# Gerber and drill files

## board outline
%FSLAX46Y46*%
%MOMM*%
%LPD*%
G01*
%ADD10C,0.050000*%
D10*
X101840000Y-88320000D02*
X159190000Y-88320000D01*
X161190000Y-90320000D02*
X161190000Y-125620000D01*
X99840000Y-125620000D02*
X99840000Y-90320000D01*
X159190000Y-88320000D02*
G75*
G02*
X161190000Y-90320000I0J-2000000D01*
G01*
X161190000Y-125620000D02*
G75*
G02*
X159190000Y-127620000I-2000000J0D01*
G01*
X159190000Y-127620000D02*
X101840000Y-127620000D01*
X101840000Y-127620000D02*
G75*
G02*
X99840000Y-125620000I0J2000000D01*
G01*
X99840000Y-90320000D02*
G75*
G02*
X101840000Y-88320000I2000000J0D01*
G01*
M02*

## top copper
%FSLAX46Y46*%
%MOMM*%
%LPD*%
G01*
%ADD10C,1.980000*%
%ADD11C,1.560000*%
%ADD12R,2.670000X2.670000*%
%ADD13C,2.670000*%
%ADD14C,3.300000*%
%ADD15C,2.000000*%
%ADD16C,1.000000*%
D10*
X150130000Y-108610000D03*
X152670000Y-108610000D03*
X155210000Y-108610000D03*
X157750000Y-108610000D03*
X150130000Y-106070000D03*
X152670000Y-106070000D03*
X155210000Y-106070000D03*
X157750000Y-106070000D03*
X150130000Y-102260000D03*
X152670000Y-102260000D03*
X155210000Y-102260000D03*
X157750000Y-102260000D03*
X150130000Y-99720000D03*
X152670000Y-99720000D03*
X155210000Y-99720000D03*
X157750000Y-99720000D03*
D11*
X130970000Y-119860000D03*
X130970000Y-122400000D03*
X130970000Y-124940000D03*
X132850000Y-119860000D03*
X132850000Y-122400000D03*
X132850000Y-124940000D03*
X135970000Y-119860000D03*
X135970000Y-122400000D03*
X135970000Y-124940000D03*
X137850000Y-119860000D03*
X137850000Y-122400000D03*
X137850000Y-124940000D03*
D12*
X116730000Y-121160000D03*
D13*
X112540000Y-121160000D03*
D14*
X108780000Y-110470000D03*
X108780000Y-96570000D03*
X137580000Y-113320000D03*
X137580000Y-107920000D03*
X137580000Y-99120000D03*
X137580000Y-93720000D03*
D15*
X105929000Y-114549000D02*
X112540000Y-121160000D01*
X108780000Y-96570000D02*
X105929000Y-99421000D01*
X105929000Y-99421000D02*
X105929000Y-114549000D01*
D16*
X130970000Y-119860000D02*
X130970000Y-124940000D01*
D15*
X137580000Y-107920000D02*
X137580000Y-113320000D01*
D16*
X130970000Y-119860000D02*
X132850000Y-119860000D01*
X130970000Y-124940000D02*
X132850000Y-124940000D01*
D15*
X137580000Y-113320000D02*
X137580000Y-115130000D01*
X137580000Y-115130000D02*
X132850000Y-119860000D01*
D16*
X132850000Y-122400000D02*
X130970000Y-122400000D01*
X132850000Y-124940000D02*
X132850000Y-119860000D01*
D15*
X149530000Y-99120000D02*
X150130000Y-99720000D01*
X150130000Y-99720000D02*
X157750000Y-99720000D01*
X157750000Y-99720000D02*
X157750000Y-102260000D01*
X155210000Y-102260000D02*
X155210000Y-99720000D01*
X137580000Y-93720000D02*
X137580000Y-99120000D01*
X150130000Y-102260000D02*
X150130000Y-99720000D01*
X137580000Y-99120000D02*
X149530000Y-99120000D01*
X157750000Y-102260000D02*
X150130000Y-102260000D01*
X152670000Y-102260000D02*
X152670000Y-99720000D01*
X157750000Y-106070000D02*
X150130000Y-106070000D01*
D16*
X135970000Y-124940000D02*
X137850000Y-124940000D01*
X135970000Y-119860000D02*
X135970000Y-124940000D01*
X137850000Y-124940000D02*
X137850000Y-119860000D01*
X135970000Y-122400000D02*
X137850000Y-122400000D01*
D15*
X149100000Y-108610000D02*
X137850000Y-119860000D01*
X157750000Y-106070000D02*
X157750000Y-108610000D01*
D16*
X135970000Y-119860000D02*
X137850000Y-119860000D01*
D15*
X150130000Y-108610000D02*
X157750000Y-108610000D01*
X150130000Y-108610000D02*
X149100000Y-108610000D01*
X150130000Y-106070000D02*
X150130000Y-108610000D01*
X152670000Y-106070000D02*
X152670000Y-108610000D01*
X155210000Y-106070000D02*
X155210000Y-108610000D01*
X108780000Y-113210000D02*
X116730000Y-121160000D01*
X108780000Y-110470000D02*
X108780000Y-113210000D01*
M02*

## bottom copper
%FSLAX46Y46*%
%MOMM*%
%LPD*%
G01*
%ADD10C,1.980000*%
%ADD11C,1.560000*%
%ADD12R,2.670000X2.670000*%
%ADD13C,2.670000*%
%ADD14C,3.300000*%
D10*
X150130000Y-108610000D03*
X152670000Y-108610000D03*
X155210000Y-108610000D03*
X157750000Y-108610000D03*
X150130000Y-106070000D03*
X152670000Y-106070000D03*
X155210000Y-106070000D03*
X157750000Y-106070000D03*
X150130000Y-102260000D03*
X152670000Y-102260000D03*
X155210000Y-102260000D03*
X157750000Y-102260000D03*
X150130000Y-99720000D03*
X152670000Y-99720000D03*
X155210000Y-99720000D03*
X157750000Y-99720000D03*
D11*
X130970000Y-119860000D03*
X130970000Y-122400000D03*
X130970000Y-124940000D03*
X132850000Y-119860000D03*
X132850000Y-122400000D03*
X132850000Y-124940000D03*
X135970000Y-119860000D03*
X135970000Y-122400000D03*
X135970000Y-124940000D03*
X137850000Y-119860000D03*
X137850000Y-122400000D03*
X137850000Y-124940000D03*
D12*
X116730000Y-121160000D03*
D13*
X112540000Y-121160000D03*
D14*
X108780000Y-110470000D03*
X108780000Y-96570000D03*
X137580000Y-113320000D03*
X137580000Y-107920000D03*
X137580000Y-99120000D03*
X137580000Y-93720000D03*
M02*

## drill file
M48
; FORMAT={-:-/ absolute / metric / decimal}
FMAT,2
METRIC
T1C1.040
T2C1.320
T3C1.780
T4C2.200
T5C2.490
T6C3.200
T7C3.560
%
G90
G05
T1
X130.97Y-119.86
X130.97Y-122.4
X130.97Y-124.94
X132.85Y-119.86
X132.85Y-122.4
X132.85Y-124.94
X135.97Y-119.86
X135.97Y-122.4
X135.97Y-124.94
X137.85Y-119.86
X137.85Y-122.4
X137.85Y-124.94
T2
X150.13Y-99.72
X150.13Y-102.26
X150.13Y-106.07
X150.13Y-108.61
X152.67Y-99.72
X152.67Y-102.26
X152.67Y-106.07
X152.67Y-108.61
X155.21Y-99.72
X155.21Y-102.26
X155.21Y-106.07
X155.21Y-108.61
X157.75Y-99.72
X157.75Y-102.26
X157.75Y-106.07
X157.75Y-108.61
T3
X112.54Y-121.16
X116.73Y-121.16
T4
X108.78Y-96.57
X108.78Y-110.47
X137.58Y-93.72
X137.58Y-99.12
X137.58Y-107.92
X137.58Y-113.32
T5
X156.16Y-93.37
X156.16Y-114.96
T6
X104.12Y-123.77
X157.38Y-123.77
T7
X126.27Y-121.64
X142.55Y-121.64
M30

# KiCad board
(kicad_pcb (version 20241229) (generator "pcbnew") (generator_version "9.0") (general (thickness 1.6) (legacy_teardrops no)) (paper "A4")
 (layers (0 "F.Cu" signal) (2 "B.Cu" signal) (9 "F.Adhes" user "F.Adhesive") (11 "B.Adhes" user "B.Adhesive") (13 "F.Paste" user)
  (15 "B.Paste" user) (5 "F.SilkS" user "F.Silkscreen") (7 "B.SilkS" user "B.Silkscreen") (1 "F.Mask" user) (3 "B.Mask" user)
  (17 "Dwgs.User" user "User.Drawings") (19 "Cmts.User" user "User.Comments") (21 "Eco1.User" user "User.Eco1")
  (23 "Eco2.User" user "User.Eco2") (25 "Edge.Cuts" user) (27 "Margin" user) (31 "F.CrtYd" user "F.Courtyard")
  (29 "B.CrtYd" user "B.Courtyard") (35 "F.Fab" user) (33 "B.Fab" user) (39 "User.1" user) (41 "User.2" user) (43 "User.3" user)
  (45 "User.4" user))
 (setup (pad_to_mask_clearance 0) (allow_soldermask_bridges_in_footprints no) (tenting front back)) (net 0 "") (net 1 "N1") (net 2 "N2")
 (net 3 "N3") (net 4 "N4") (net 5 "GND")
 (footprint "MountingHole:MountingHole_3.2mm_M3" (layer "F.Cu") (at 104.12 123.77)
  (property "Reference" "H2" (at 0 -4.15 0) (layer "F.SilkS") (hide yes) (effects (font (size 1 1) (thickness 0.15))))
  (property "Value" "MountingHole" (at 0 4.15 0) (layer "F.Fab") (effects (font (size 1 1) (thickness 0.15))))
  (pad "" np_thru_hole circle (at 0 0) (size 3.2 3.2) (drill 3.2) (layers "*.Cu" "*.Mask")))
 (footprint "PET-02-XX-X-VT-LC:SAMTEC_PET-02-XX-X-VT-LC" (layer "F.Cu") (at 154.16 104.31 90)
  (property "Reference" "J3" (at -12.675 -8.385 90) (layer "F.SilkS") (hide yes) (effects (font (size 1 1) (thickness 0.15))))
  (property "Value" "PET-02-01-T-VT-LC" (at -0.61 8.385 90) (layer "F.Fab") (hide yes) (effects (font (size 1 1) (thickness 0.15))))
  (pad "" np_thru_hole circle (at -10.65 2 90) (size 2.49 2.49) (drill 2.49) (layers "*.Cu" "*.Mask"))
  (pad "" np_thru_hole circle (at 10.94 2 90) (size 2.49 2.49) (drill 2.49) (layers "*.Cu" "*.Mask"))
  (pad "1" thru_hole circle (at -4.3 -4.03 90) (size 1.98 1.98) (drill 1.32) (layers "*.Cu" "*.Mask") (remove_unused_layers no) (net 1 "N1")
   (solder_mask_margin 0.102))
  (pad "1" thru_hole circle (at -4.3 -1.49 90) (size 1.98 1.98) (drill 1.32) (layers "*.Cu" "*.Mask") (remove_unused_layers no) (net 1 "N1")
   (solder_mask_margin 0.102))
  (pad "1" thru_hole circle (at -4.3 1.05 90) (size 1.98 1.98) (drill 1.32) (layers "*.Cu" "*.Mask") (remove_unused_layers no) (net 1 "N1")
   (solder_mask_margin 0.102))
  (pad "1" thru_hole circle (at -4.3 3.59 90) (size 1.98 1.98) (drill 1.32) (layers "*.Cu" "*.Mask") (remove_unused_layers no) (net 1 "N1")
   (solder_mask_margin 0.102))
  (pad "1" thru_hole circle (at -1.76 -4.03 90) (size 1.98 1.98) (drill 1.32) (layers "*.Cu" "*.Mask") (remove_unused_layers no)
   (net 1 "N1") (solder_mask_margin 0.102))
  (pad "1" thru_hole circle (at -1.76 -1.49 90) (size 1.98 1.98) (drill 1.32) (layers "*.Cu" "*.Mask") (remove_unused_layers no)
   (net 1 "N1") (solder_mask_margin 0.102))
  (pad "1" thru_hole circle (at -1.76 1.05 90) (size 1.98 1.98) (drill 1.32) (layers "*.Cu" "*.Mask") (remove_unused_layers no) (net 1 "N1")
   (solder_mask_margin 0.102))
  (pad "1" thru_hole circle (at -1.76 3.59 90) (size 1.98 1.98) (drill 1.32) (layers "*.Cu" "*.Mask") (remove_unused_layers no) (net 1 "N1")
   (solder_mask_margin 0.102))
  (pad "2" thru_hole circle (at 2.05 -4.03 90) (size 1.98 1.98) (drill 1.32) (layers "*.Cu" "*.Mask") (remove_unused_layers no) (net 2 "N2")
   (solder_mask_margin 0.102))
  (pad "2" thru_hole circle (at 2.05 -1.49 90) (size 1.98 1.98) (drill 1.32) (layers "*.Cu" "*.Mask") (remove_unused_layers no) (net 2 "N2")
   (solder_mask_margin 0.102))
  (pad "2" thru_hole circle (at 2.05 1.05 90) (size 1.98 1.98) (drill 1.32) (layers "*.Cu" "*.Mask") (remove_unused_layers no) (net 2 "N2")
   (solder_mask_margin 0.102))
  (pad "2" thru_hole circle (at 2.05 3.59 90) (size 1.98 1.98) (drill 1.32) (layers "*.Cu" "*.Mask") (remove_unused_layers no) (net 2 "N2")
   (solder_mask_margin 0.102))
  (pad "2" thru_hole circle (at 4.59 -4.03 90) (size 1.98 1.98) (drill 1.32) (layers "*.Cu" "*.Mask") (remove_unused_layers no) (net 2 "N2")
   (solder_mask_margin 0.102))
  (pad "2" thru_hole circle (at 4.59 -1.49 90) (size 1.98 1.98) (drill 1.32) (layers "*.Cu" "*.Mask") (remove_unused_layers no) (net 2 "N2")
   (solder_mask_margin 0.102))
  (pad "2" thru_hole circle (at 4.59 1.05 90) (size 1.98 1.98) (drill 1.32) (layers "*.Cu" "*.Mask") (remove_unused_layers no) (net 2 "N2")
   (solder_mask_margin 0.102))
  (pad "2" thru_hole circle (at 4.59 3.59 90) (size 1.98 1.98) (drill 1.32) (layers "*.Cu" "*.Mask") (remove_unused_layers no) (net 2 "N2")
   (solder_mask_margin 0.102)))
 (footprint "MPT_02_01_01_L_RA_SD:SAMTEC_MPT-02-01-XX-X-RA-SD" (layer "F.Cu") (at 134.41 127.79)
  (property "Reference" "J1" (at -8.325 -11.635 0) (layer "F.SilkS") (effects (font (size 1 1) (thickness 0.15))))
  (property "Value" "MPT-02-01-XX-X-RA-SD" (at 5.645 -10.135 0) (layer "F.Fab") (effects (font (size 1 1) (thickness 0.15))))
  (pad "" np_thru_hole circle (at -8.14 -6.15) (size 3.56 3.56) (drill 3.56) (layers "*.Cu" "*.Mask"))
  (pad "" np_thru_hole circle (at 8.14 -6.15) (size 3.56 3.56) (drill 3.56) (layers "*.Cu" "*.Mask"))
  (pad "1" thru_hole circle (at -3.44 -7.93) (size 1.56 1.56) (drill 1.04) (layers "*.Cu" "*.Mask") (remove_unused_layers no) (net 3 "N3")
   (solder_mask_margin 0.102))
  (pad "1" thru_hole circle (at -3.44 -5.39) (size 1.56 1.56) (drill 1.04) (layers "*.Cu" "*.Mask") (remove_unused_layers no) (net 3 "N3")
   (solder_mask_margin 0.102))
  (pad "1" thru_hole circle (at -3.44 -2.85) (size 1.56 1.56) (drill 1.04) (layers "*.Cu" "*.Mask") (remove_unused_layers no) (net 3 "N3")
   (solder_mask_margin 0.102))
  (pad "1" thru_hole circle (at -1.56 -7.93) (size 1.56 1.56) (drill 1.04) (layers "*.Cu" "*.Mask") (remove_unused_layers no) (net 3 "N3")
   (solder_mask_margin 0.102))
  (pad "1" thru_hole circle (at -1.56 -5.39) (size 1.56 1.56) (drill 1.04) (layers "*.Cu" "*.Mask") (remove_unused_layers no) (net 3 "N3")
   (solder_mask_margin 0.102))
  (pad "1" thru_hole circle (at -1.56 -2.85) (size 1.56 1.56) (drill 1.04) (layers "*.Cu" "*.Mask") (remove_unused_layers no) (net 3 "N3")
   (solder_mask_margin 0.102))
  (pad "2" thru_hole circle (at 1.56 -7.93) (size 1.56 1.56) (drill 1.04) (layers "*.Cu" "*.Mask") (remove_unused_layers no) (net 1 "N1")
   (solder_mask_margin 0.102))
  (pad "2" thru_hole circle (at 1.56 -5.39) (size 1.56 1.56) (drill 1.04) (layers "*.Cu" "*.Mask") (remove_unused_layers no) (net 1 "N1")
   (solder_mask_margin 0.102))
  (pad "2" thru_hole circle (at 1.56 -2.85) (size 1.56 1.56) (drill 1.04) (layers "*.Cu" "*.Mask") (remove_unused_layers no) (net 1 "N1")
   (solder_mask_margin 0.102))
  (pad "2" thru_hole circle (at 3.44 -7.93) (size 1.56 1.56) (drill 1.04) (layers "*.Cu" "*.Mask") (remove_unused_layers no) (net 1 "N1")
   (solder_mask_margin 0.102))
  (pad "2" thru_hole circle (at 3.44 -5.39) (size 1.56 1.56) (drill 1.04) (layers "*.Cu" "*.Mask") (remove_unused_layers no) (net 1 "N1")
   (solder_mask_margin 0.102))
  (pad "2" thru_hole circle (at 3.44 -2.85) (size 1.56 1.56) (drill 1.04) (layers "*.Cu" "*.Mask") (remove_unused_layers no) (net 1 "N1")
   (solder_mask_margin 0.102)))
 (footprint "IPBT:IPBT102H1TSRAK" (layer "F.Cu") (at 116.73 121.16 180)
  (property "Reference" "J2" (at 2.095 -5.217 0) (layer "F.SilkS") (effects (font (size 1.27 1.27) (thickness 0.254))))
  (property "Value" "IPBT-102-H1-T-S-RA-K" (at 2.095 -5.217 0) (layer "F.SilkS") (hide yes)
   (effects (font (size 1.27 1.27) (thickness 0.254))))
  (pad "1" thru_hole rect (at 0 0 180) (size 2.67 2.67) (drill 1.78) (layers "*.Cu" "*.Mask") (remove_unused_layers no) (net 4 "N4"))
  (pad "2" thru_hole circle (at 4.19 0 180) (size 2.67 2.67) (drill 1.78) (layers "*.Cu" "*.Mask") (remove_unused_layers no) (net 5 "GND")))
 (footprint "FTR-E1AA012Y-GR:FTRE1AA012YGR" (layer "F.Cu") (at 108.78 110.47)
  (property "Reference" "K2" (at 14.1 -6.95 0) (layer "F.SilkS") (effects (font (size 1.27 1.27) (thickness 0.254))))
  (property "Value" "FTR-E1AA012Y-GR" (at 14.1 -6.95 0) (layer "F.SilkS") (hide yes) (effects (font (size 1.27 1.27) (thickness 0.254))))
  (pad "1" thru_hole circle (at 0 0) (size 3.3 3.3) (drill 2.2) (layers "*.Cu" "*.Mask") (remove_unused_layers no) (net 4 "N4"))
  (pad "2" thru_hole circle (at 0 -13.9) (size 3.3 3.3) (drill 2.2) (layers "*.Cu" "*.Mask") (remove_unused_layers no) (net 5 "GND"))
  (pad "31" thru_hole circle (at 28.8 2.85) (size 3.3 3.3) (drill 2.2) (layers "*.Cu" "*.Mask") (remove_unused_layers no) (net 3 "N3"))
  (pad "32" thru_hole circle (at 28.8 -2.55) (size 3.3 3.3) (drill 2.2) (layers "*.Cu" "*.Mask") (remove_unused_layers no) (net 3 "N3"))
  (pad "41" thru_hole circle (at 28.8 -11.35) (size 3.3 3.3) (drill 2.2) (layers "*.Cu" "*.Mask") (remove_unused_layers no) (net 2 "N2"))
  (pad "42" thru_hole circle (at 28.8 -16.75) (size 3.3 3.3) (drill 2.2) (layers "*.Cu" "*.Mask") (remove_unused_layers no) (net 2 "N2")))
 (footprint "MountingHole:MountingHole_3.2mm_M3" (layer "F.Cu") (at 157.38 123.77)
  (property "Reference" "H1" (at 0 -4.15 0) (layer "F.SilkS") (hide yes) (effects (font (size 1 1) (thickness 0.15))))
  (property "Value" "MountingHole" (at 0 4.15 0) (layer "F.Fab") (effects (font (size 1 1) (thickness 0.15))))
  (pad "" np_thru_hole circle (at 0 0) (size 3.2 3.2) (drill 3.2) (layers "*.Cu" "*.Mask")))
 (gr_line (start 101.84 88.32) (end 159.19 88.32) (stroke (width 0.05) (type default)) (layer "Edge.Cuts"))
 (gr_line (start 161.19 90.32) (end 161.19 125.62) (stroke (width 0.05) (type default)) (layer "Edge.Cuts"))
 (gr_line (start 99.84 125.62) (end 99.84 90.32) (stroke (width 0.05) (type default)) (layer "Edge.Cuts"))
 (gr_arc (start 159.19 88.32) (mid 160.604214 88.905786) (end 161.19 90.32) (stroke (width 0.05) (type default)) (layer "Edge.Cuts"))
 (gr_arc (start 161.19 125.62) (mid 160.604214 127.034214) (end 159.19 127.62) (stroke (width 0.05) (type default)) (layer "Edge.Cuts"))
 (gr_line (start 159.19 127.62) (end 101.84 127.62) (stroke (width 0.05) (type default)) (layer "Edge.Cuts"))
 (gr_arc (start 101.84 127.62) (mid 100.425786 127.034214) (end 99.84 125.62) (stroke (width 0.05) (type default)) (layer "Edge.Cuts"))
 (gr_arc (start 99.84 90.32) (mid 100.425786 88.905786) (end 101.84 88.32) (stroke (width 0.05) (type default)) (layer "Edge.Cuts"))
 (segment (start 105.929 114.549) (end 112.54 121.16) (width 2) (layer "F.Cu") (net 5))
 (segment (start 108.78 96.57) (end 105.929 99.421) (width 2) (layer "F.Cu") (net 5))
 (segment (start 105.929 99.421) (end 105.929 114.549) (width 2) (layer "F.Cu") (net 5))
 (segment (start 130.97 119.86) (end 130.97 124.94) (width 1) (layer "F.Cu") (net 3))
 (segment (start 137.58 107.92) (end 137.58 113.32) (width 2) (layer "F.Cu") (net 3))
 (segment (start 130.97 119.86) (end 132.85 119.86) (width 1) (layer "F.Cu") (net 3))
 (segment (start 130.97 124.94) (end 132.85 124.94) (width 1) (layer "F.Cu") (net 3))
 (segment (start 137.58 113.32) (end 137.58 115.13) (width 2) (layer "F.Cu") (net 3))
 (segment (start 137.58 115.13) (end 132.85 119.86) (width 2) (layer "F.Cu") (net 3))
 (segment (start 132.85 122.4) (end 130.97 122.4) (width 1) (layer "F.Cu") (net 3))
 (segment (start 132.85 124.94) (end 132.85 119.86) (width 1) (layer "F.Cu") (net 3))
 (segment (start 149.53 99.12) (end 150.13 99.72) (width 2) (layer "F.Cu") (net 2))
 (segment (start 150.13 99.72) (end 157.75 99.72) (width 2) (layer "F.Cu") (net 2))
 (segment (start 157.75 99.72) (end 157.75 102.26) (width 2) (layer "F.Cu") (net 2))
 (segment (start 155.21 102.26) (end 155.21 99.72) (width 2) (layer "F.Cu") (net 2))
 (segment (start 137.58 93.72) (end 137.58 99.12) (width 2) (layer "F.Cu") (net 2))
 (segment (start 150.13 102.26) (end 150.13 99.72) (width 2) (layer "F.Cu") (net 2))
 (segment (start 137.58 99.12) (end 149.53 99.12) (width 2) (layer "F.Cu") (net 2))
 (segment (start 157.75 102.26) (end 150.13 102.26) (width 2) (layer "F.Cu") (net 2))
 (segment (start 152.67 102.26) (end 152.67 99.72) (width 2) (layer "F.Cu") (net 2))
 (segment (start 157.75 106.07) (end 150.13 106.07) (width 2) (layer "F.Cu") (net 1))
 (segment (start 135.97 124.94) (end 137.85 124.94) (width 1) (layer "F.Cu") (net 1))
 (segment (start 135.97 119.86) (end 135.97 124.94) (width 1) (layer "F.Cu") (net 1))
 (segment (start 137.85 124.94) (end 137.85 119.86) (width 1) (layer "F.Cu") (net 1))
 (segment (start 135.97 122.4) (end 137.85 122.4) (width 1) (layer "F.Cu") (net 1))
 (segment (start 149.1 108.61) (end 137.85 119.86) (width 2) (layer "F.Cu") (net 1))
 (segment (start 157.75 106.07) (end 157.75 108.61) (width 2) (layer "F.Cu") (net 1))
 (segment (start 135.97 119.86) (end 137.85 119.86) (width 1) (layer "F.Cu") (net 1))
 (segment (start 150.13 108.61) (end 157.75 108.61) (width 2) (layer "F.Cu") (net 1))
 (segment (start 150.13 108.61) (end 149.1 108.61) (width 2) (layer "F.Cu") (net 1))
 (segment (start 150.13 106.07) (end 150.13 108.61) (width 2) (layer "F.Cu") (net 1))
 (segment (start 152.67 106.07) (end 152.67 108.61) (width 2) (layer "F.Cu") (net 1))
 (segment (start 155.21 106.07) (end 155.21 108.61) (width 2) (layer "F.Cu") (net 1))
 (segment (start 108.78 113.21) (end 116.73 121.16) (width 2) (layer "F.Cu") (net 4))
 (segment (start 108.78 110.47) (end 108.78 113.21) (width 2) (layer "F.Cu") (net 4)))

